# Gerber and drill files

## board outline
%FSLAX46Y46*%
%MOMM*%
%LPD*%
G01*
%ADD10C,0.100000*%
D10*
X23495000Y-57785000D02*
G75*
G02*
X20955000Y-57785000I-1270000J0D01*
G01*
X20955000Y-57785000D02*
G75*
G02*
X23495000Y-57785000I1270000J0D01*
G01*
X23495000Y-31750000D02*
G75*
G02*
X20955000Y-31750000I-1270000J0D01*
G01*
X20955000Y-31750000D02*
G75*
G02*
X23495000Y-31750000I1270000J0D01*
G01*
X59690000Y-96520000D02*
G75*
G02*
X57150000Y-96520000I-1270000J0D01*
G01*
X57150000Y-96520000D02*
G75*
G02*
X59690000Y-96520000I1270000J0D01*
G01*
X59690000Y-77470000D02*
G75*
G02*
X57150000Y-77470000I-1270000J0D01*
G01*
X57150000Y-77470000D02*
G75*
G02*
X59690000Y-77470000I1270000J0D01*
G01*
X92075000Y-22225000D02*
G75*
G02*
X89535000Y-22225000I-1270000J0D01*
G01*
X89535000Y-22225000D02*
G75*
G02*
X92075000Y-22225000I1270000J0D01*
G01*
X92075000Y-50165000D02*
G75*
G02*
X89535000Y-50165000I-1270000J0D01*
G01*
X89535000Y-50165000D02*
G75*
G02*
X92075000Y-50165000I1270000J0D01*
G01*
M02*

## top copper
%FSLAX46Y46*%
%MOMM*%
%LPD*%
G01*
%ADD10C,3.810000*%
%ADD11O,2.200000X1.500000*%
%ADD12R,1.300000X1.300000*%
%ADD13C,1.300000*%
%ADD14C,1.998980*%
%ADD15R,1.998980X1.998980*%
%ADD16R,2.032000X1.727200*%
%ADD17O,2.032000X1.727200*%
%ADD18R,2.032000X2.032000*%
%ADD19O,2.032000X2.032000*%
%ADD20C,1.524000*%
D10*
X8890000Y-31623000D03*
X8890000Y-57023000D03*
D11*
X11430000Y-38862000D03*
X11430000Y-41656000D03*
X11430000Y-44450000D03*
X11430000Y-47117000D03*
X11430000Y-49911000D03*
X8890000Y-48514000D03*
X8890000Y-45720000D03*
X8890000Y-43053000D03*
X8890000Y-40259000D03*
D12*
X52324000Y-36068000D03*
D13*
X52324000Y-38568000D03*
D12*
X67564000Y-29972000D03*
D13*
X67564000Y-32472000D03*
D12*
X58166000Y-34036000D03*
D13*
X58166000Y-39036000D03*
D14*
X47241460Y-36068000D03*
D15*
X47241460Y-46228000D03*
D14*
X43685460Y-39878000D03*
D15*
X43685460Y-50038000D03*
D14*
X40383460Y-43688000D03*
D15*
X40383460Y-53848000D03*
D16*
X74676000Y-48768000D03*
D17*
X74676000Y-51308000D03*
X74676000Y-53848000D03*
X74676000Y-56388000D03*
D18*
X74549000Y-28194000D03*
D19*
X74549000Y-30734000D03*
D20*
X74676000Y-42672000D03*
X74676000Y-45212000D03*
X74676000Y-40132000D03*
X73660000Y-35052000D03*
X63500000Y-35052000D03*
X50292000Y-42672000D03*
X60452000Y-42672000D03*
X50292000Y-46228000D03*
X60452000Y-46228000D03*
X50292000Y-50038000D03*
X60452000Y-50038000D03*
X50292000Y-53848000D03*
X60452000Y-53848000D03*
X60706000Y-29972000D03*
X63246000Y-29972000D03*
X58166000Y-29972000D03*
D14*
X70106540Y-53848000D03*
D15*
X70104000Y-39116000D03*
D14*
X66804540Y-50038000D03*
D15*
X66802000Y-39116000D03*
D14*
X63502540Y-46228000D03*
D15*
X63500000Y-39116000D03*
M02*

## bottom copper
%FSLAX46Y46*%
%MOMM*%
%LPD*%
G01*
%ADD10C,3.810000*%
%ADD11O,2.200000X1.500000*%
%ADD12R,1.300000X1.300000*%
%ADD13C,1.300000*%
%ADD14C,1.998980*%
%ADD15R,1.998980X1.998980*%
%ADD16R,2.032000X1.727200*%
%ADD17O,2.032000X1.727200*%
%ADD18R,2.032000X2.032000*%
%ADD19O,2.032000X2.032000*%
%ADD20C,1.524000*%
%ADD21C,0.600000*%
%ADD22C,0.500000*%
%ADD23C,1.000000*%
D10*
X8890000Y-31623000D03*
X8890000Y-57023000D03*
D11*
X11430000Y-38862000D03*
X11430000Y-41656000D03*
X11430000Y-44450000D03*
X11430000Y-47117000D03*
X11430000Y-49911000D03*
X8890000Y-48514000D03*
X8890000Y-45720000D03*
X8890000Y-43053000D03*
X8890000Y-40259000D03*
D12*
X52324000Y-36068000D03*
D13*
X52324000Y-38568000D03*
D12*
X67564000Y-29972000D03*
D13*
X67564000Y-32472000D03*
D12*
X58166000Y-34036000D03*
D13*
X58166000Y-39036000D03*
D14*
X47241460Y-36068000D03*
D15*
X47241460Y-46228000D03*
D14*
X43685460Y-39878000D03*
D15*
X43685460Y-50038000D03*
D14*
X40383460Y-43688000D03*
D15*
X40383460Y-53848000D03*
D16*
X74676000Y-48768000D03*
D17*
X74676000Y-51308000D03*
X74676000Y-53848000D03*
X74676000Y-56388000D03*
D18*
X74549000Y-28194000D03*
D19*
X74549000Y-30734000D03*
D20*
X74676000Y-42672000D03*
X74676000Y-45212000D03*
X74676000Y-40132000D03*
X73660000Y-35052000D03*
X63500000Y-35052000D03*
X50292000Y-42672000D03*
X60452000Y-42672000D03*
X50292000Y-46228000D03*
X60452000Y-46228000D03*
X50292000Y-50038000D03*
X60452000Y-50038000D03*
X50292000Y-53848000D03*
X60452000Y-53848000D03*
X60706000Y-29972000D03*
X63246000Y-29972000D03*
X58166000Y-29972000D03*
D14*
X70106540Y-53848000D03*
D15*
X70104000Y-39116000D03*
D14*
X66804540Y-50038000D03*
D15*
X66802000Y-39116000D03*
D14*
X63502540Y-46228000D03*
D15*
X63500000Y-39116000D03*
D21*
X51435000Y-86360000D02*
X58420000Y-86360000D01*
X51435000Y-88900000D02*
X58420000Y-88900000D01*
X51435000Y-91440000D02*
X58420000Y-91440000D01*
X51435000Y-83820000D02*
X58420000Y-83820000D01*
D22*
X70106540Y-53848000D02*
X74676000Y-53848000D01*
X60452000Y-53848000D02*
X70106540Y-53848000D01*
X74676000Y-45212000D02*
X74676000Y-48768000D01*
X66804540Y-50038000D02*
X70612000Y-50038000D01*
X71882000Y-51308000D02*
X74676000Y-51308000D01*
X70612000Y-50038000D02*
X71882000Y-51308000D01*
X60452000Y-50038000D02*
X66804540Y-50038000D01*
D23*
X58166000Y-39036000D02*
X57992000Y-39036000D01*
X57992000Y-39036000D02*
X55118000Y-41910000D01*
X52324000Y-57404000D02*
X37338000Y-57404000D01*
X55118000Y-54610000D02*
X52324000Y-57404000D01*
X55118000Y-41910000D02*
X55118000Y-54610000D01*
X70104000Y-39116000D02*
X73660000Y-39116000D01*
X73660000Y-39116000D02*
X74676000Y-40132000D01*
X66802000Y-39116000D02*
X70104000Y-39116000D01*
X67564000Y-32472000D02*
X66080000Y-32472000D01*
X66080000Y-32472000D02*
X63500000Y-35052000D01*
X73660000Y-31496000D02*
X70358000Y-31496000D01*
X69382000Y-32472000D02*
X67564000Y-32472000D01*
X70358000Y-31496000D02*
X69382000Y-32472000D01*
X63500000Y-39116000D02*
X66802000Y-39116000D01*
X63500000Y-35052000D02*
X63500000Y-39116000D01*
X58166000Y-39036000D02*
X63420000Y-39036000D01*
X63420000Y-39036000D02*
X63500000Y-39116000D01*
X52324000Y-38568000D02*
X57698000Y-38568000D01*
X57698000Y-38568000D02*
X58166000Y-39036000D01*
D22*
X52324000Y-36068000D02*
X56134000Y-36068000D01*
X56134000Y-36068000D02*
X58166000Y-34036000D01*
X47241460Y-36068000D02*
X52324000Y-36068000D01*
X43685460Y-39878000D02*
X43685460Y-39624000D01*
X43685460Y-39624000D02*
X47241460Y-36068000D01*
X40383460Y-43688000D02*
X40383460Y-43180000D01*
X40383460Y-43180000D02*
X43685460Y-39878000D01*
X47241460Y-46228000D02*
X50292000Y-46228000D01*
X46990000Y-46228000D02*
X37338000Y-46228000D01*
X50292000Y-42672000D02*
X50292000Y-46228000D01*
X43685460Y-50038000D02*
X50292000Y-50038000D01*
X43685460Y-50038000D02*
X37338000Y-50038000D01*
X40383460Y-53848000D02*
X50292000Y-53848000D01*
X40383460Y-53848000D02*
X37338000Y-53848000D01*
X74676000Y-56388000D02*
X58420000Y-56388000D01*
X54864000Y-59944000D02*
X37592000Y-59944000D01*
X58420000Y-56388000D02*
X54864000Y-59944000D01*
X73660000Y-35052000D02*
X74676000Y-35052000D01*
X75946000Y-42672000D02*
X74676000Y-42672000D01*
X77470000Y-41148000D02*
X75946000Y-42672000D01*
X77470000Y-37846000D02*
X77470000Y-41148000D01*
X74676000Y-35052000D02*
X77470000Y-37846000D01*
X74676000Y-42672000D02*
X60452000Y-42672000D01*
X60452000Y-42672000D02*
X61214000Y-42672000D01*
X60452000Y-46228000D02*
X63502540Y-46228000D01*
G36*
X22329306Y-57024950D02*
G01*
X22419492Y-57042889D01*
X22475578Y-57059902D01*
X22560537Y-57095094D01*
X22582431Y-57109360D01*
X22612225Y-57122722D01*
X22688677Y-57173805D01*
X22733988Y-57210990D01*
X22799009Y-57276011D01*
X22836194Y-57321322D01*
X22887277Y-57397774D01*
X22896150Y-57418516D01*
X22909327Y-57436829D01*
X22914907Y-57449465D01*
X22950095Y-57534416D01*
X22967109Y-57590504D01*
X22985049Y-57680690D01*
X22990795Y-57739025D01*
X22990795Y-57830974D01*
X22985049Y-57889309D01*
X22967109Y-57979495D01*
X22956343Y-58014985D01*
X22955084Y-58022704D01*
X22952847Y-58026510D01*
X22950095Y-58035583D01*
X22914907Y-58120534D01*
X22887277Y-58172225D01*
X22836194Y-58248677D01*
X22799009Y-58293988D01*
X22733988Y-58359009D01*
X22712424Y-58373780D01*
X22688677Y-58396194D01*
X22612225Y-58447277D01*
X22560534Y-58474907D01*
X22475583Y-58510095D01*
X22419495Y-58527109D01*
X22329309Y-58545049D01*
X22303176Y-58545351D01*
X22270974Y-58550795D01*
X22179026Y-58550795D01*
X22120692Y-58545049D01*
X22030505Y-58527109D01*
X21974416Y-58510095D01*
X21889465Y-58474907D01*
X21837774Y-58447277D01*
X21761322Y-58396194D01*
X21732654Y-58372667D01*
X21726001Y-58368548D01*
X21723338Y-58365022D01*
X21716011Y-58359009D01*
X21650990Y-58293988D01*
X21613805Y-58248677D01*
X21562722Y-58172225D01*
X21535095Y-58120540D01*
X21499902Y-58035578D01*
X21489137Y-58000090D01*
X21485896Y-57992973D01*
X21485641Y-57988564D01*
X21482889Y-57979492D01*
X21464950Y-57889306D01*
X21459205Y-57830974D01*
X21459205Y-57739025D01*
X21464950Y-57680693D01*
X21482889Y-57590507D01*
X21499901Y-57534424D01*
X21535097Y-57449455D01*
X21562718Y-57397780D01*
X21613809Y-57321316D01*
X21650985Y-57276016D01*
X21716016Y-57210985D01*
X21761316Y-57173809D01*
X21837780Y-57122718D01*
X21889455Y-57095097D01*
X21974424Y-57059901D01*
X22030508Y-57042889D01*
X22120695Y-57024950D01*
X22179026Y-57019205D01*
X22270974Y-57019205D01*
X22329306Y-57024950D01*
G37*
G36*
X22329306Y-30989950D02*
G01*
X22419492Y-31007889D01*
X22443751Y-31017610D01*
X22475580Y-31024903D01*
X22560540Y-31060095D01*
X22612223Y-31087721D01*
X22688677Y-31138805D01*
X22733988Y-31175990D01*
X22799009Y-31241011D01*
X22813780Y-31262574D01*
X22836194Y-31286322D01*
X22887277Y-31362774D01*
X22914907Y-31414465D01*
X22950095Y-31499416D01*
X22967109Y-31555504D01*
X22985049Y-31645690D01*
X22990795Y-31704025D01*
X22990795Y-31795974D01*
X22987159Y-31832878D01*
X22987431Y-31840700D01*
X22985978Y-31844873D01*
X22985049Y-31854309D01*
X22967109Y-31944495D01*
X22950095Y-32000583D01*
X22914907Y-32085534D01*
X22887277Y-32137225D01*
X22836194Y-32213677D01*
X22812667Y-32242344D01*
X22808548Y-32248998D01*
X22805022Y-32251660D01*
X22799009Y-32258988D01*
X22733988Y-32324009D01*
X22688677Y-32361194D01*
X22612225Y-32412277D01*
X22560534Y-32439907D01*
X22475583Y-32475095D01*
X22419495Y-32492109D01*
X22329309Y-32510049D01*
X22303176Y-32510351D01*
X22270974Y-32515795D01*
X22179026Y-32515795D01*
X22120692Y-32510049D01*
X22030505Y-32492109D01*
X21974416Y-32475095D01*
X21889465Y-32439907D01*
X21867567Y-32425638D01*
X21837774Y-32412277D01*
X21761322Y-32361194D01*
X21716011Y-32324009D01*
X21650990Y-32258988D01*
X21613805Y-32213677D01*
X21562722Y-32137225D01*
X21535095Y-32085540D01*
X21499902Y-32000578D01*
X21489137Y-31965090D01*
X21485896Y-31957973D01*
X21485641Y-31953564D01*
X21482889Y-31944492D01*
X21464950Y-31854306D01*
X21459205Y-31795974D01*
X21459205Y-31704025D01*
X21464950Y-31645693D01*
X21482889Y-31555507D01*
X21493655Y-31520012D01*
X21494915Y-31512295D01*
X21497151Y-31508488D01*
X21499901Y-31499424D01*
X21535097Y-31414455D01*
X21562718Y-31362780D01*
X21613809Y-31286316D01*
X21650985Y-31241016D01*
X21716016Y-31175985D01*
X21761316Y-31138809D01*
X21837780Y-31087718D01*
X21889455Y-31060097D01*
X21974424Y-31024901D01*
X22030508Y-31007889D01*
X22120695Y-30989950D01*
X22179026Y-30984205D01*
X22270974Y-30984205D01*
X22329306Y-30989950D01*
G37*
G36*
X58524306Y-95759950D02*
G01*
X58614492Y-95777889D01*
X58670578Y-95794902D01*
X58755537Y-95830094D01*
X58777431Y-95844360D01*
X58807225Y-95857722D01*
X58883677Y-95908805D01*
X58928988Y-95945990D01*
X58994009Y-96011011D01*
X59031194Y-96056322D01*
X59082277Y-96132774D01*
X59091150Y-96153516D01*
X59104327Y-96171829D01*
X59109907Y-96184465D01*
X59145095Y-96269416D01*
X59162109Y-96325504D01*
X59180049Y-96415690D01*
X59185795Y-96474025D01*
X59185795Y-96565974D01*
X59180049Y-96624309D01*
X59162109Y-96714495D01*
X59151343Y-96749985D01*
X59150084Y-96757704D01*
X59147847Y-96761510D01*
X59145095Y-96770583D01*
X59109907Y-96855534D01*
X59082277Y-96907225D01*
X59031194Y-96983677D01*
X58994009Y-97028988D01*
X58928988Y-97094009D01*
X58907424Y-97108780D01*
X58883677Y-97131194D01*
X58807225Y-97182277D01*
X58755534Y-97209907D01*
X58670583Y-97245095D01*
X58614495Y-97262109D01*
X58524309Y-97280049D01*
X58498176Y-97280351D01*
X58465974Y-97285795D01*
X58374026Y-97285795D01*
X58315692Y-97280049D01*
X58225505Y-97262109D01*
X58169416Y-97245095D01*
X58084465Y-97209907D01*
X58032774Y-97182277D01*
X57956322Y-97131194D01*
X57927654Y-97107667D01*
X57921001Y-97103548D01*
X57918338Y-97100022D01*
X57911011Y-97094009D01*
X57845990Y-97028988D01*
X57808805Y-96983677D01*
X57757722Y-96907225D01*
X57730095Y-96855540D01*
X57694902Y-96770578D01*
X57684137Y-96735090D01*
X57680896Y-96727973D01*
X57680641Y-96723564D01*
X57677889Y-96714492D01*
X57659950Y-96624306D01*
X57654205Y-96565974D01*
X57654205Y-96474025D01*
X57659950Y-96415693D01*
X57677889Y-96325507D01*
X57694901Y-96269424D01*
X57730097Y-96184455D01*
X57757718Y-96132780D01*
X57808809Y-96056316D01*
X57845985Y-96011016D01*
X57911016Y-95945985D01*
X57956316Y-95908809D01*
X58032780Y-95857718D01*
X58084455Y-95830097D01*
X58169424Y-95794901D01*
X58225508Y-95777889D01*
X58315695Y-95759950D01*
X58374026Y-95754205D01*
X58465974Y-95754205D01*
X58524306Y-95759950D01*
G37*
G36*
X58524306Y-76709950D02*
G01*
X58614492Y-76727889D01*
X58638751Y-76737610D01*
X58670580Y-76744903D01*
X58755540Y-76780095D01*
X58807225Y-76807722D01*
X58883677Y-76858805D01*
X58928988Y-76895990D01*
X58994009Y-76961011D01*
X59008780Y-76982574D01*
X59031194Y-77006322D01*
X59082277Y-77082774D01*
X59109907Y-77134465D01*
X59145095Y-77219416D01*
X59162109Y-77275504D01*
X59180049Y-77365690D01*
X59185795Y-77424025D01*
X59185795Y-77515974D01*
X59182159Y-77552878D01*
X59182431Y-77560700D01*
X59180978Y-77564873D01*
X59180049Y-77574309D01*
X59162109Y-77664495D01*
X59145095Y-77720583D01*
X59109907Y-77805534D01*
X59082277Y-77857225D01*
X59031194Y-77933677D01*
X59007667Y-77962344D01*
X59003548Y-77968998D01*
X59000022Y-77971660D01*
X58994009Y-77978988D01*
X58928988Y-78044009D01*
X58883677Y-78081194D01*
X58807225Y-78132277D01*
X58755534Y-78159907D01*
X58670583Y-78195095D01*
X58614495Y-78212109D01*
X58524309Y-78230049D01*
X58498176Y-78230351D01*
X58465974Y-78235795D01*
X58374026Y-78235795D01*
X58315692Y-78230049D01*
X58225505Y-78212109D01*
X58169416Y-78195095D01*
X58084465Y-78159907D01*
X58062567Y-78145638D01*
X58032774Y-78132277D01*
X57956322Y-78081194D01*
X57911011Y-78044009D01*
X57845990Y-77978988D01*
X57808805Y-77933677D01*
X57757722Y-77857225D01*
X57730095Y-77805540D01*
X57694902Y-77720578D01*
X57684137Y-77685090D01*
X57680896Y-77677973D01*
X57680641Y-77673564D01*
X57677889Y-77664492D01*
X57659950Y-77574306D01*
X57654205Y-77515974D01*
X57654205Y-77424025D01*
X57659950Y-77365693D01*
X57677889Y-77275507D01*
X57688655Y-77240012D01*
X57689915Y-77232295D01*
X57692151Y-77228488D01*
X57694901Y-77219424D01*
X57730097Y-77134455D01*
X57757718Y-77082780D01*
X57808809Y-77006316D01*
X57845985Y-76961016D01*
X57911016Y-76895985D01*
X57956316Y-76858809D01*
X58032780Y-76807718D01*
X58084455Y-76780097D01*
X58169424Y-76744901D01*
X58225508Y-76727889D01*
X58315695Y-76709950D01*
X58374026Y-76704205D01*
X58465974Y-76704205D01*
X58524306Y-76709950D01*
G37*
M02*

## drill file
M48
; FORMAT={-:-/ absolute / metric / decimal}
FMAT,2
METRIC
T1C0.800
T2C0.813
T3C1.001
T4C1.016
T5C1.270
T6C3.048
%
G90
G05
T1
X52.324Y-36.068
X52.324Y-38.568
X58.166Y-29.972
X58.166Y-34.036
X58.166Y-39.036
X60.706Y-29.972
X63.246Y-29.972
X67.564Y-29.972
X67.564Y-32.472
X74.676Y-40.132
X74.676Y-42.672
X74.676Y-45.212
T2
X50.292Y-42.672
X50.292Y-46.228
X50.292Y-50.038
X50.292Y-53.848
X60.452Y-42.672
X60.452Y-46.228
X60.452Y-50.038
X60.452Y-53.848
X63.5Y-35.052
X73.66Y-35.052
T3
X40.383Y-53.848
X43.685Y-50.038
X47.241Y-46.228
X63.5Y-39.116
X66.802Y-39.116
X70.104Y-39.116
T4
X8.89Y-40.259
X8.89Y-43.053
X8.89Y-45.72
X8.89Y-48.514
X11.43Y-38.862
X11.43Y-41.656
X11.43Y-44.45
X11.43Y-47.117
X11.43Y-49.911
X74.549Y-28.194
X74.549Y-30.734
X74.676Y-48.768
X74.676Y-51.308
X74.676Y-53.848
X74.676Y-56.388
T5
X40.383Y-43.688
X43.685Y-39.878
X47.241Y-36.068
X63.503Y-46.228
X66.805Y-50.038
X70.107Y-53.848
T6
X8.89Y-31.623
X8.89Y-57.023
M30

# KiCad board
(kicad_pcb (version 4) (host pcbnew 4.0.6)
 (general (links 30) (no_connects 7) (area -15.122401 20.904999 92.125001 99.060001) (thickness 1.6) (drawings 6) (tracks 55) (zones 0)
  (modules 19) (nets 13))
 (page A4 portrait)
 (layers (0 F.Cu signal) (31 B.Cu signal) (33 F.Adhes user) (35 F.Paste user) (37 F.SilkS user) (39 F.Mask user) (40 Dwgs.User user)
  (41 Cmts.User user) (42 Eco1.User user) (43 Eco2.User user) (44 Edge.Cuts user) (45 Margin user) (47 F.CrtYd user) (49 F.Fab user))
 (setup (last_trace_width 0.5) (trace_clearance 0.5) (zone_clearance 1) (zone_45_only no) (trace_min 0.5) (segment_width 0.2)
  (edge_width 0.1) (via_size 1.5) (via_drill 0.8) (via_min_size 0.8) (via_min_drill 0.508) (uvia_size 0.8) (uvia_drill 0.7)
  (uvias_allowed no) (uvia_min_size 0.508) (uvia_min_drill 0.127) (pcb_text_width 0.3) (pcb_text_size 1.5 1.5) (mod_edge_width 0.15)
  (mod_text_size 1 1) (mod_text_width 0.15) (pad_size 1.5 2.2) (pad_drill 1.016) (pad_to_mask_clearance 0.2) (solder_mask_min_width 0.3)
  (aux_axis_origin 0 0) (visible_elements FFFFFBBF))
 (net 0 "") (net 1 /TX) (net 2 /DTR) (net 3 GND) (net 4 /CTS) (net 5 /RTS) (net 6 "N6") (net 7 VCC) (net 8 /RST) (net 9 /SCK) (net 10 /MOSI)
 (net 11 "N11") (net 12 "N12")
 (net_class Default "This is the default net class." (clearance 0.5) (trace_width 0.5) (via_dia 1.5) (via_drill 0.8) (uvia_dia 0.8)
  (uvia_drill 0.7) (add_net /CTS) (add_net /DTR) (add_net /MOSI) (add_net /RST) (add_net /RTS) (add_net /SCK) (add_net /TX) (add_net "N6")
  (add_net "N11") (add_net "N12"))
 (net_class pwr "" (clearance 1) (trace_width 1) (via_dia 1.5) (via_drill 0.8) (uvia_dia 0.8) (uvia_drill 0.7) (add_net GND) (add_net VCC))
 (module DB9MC (layer F.Cu) (at 10.16 44.45 90)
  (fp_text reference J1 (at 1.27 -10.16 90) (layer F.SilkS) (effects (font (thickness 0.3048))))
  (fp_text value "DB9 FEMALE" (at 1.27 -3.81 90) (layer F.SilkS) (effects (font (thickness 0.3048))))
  (pad "" thru_hole circle (at 12.827 -1.27 90) (size 3.81 3.81) (drill 3.048) (layers *.Cu *.Mask F.SilkS))
  (pad "" thru_hole circle (at -12.573 -1.27 90) (size 3.81 3.81) (drill 3.048) (layers *.Cu *.Mask F.SilkS))
  (pad 1 thru_hole oval (at 5.588 1.27 90) (size 1.5 2.2) (drill 1.016) (layers *.Cu *.Mask F.SilkS))
  (pad 2 thru_hole oval (at 2.794 1.27 90) (size 1.5 2.2) (drill 1.016) (layers *.Cu *.Mask F.SilkS))
  (pad 3 thru_hole oval (at 0 1.27 90) (size 1.5 2.2) (drill 1.016) (layers *.Cu *.Mask F.SilkS) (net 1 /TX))
  (pad 4 thru_hole oval (at -2.667 1.27 90) (size 1.5 2.2) (drill 1.016) (layers *.Cu *.Mask F.SilkS) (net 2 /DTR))
  (pad 5 thru_hole oval (at -5.461 1.27 90) (size 1.5 2.2) (drill 1.016) (layers *.Cu *.Mask F.SilkS) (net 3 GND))
  (pad 9 thru_hole oval (at -4.064 -1.27 90) (size 1.5 2.2) (drill 1.016) (layers *.Cu *.Mask F.SilkS))
  (pad 8 thru_hole oval (at -1.27 -1.27 90) (size 1.5 2.2) (drill 1.016) (layers *.Cu *.Mask F.SilkS) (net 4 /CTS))
  (pad 7 thru_hole oval (at 1.397 -1.27 90) (size 1.5 2.2) (drill 1.016) (layers *.Cu *.Mask F.SilkS) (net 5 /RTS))
  (pad 6 thru_hole oval (at 4.191 -1.27 90) (size 1.5 2.2) (drill 1.016) (layers *.Cu *.Mask F.SilkS)))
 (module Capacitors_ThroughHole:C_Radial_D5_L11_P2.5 (layer F.Cu) (at 52.324 36.068 270)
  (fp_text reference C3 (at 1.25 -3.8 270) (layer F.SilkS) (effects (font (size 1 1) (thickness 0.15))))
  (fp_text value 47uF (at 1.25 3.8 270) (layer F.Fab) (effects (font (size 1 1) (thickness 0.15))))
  (pad 1 thru_hole rect (at 0 0 270) (size 1.3 1.3) (drill 0.8) (layers *.Cu *.Mask F.SilkS) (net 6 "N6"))
  (pad 2 thru_hole circle (at 2.5 0 270) (size 1.3 1.3) (drill 0.8) (layers *.Cu *.Mask F.SilkS) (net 3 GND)))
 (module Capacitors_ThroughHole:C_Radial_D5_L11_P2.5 (layer F.Cu) (at 67.564 29.972 270)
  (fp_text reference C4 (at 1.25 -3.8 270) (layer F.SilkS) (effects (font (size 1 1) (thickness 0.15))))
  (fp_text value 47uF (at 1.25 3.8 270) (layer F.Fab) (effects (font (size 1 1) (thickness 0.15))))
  (pad 1 thru_hole rect (at 0 0 270) (size 1.3 1.3) (drill 0.8) (layers *.Cu *.Mask F.SilkS) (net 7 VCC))
  (pad 2 thru_hole circle (at 2.5 0 270) (size 1.3 1.3) (drill 0.8) (layers *.Cu *.Mask F.SilkS) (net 3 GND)))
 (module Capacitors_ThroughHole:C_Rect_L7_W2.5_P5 (layer F.Cu) (at 58.166 34.036 270)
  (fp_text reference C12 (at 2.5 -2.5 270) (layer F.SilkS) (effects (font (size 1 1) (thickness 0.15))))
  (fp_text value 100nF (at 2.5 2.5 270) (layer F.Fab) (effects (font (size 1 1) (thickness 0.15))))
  (pad 1 thru_hole rect (at 0 0 270) (size 1.3 1.3) (drill 0.8) (layers *.Cu *.Mask F.SilkS) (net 6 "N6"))
  (pad 2 thru_hole circle (at 5 0 270) (size 1.3 1.3) (drill 0.8) (layers *.Cu *.Mask F.SilkS) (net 3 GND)))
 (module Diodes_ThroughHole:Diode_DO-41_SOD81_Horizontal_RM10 (layer F.Cu) (at 47.244 46.228 90)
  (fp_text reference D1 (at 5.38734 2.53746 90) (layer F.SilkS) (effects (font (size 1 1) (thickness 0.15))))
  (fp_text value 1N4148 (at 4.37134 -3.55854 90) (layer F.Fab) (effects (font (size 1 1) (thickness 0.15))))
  (pad 2 thru_hole circle (at 10.16 -0.00254 270) (size 1.99898 1.99898) (drill 1.27) (layers *.Cu *.Mask F.SilkS) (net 6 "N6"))
  (pad 1 thru_hole rect (at 0 -0.00254 270) (size 1.99898 1.99898) (drill 1.00076) (layers *.Cu *.Mask F.SilkS) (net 1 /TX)))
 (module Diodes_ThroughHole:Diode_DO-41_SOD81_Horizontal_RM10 (layer F.Cu) (at 43.688 50.038 90)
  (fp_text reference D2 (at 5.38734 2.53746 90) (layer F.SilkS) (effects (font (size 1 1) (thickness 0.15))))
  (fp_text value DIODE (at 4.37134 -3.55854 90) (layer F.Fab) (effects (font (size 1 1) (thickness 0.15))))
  (pad 2 thru_hole circle (at 10.16 -0.00254 270) (size 1.99898 1.99898) (drill 1.27) (layers *.Cu *.Mask F.SilkS) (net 6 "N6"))
  (pad 1 thru_hole rect (at 0 -0.00254 270) (size 1.99898 1.99898) (drill 1.00076) (layers *.Cu *.Mask F.SilkS) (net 5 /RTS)))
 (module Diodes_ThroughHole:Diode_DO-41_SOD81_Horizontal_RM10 (layer F.Cu) (at 40.386 53.848 90)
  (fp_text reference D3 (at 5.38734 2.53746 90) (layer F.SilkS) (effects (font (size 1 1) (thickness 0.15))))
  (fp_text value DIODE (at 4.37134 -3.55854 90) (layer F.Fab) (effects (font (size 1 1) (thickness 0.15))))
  (pad 2 thru_hole circle (at 10.16 -0.00254 270) (size 1.99898 1.99898) (drill 1.27) (layers *.Cu *.Mask F.SilkS) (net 6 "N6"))
  (pad 1 thru_hole rect (at 0 -0.00254 270) (size 1.99898 1.99898) (drill 1.00076) (layers *.Cu *.Mask F.SilkS) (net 2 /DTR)))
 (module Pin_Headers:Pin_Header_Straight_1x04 (layer F.Cu) (at 74.676 48.768)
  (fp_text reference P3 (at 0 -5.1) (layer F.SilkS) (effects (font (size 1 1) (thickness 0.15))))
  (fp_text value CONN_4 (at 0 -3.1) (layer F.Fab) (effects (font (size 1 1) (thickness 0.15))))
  (pad 1 thru_hole rect (at 0 0) (size 2.032 1.7272) (drill 1.016) (layers *.Cu *.Mask F.SilkS) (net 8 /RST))
  (pad 2 thru_hole oval (at 0 2.54) (size 2.032 1.7272) (drill 1.016) (layers *.Cu *.Mask F.SilkS) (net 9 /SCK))
  (pad 3 thru_hole oval (at 0 5.08) (size 2.032 1.7272) (drill 1.016) (layers *.Cu *.Mask F.SilkS) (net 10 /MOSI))
  (pad 4 thru_hole oval (at 0 7.62) (size 2.032 1.7272) (drill 1.016) (layers *.Cu *.Mask F.SilkS) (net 4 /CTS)))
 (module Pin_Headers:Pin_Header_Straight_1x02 (layer F.Cu) (at 74.549 28.194)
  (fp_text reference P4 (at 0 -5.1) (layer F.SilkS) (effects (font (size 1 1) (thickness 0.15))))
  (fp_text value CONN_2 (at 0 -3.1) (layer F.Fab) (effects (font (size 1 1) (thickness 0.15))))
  (pad 1 thru_hole rect (at 0 0) (size 2.032 2.032) (drill 1.016) (layers *.Cu *.Mask F.SilkS) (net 7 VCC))
  (pad 2 thru_hole oval (at 0 2.54) (size 2.032 2.032) (drill 1.016) (layers *.Cu *.Mask F.SilkS) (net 3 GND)))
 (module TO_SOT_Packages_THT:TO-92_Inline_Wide (layer F.Cu) (at 74.676 40.132 270)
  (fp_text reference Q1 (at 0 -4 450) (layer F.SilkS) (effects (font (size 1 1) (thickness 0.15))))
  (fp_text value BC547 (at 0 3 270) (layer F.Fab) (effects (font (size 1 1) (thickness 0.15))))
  (pad 2 thru_hole circle (at 2.54 0) (size 1.524 1.524) (drill 0.8) (layers *.Cu *.Mask F.SilkS) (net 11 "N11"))
  (pad 3 thru_hole circle (at 5.08 0) (size 1.524 1.524) (drill 0.8) (layers *.Cu *.Mask F.SilkS) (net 8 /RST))
  (pad 1 thru_hole circle (at 0 0) (size 1.524 1.524) (drill 0.8) (layers *.Cu *.Mask F.SilkS) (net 3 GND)))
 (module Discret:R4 (layer F.Cu) (at 68.58 35.052 180)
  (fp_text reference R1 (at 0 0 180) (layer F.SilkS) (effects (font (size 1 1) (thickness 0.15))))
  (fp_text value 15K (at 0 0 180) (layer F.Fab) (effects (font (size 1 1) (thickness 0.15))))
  (pad 1 thru_hole circle (at -5.08 0 180) (size 1.524 1.524) (drill 0.8128) (layers *.Cu *.Mask F.SilkS) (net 11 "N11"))
  (pad 2 thru_hole circle (at 5.08 0 180) (size 1.524 1.524) (drill 0.8128) (layers *.Cu *.Mask F.SilkS) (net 3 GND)))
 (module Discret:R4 (layer F.Cu) (at 55.372 42.672)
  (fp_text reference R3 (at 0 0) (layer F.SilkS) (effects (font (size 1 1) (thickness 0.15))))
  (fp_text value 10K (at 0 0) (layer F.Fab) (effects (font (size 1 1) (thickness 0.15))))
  (pad 1 thru_hole circle (at -5.08 0) (size 1.524 1.524) (drill 0.8128) (layers *.Cu *.Mask F.SilkS) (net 1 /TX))
  (pad 2 thru_hole circle (at 5.08 0) (size 1.524 1.524) (drill 0.8128) (layers *.Cu *.Mask F.SilkS) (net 11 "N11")))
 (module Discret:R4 (layer F.Cu) (at 55.372 46.228)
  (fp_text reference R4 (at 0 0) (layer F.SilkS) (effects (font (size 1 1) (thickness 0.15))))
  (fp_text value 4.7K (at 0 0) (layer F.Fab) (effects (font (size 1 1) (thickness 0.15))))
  (pad 1 thru_hole circle (at -5.08 0) (size 1.524 1.524) (drill 0.8128) (layers *.Cu *.Mask F.SilkS) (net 1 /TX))
  (pad 2 thru_hole circle (at 5.08 0) (size 1.524 1.524) (drill 0.8128) (layers *.Cu *.Mask F.SilkS) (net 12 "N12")))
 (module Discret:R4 (layer F.Cu) (at 55.372 50.038)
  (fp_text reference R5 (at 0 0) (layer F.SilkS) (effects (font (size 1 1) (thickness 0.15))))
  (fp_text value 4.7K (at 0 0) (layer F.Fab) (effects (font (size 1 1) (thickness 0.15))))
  (pad 1 thru_hole circle (at -5.08 0) (size 1.524 1.524) (drill 0.8128) (layers *.Cu *.Mask F.SilkS) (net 5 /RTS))
  (pad 2 thru_hole circle (at 5.08 0) (size 1.524 1.524) (drill 0.8128) (layers *.Cu *.Mask F.SilkS) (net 9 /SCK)))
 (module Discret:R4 (layer F.Cu) (at 55.372 53.848)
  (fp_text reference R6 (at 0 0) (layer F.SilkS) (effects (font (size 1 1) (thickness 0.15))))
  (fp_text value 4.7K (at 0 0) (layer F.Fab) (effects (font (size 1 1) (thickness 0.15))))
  (pad 1 thru_hole circle (at -5.08 0) (size 1.524 1.524) (drill 0.8128) (layers *.Cu *.Mask F.SilkS) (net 2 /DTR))
  (pad 2 thru_hole circle (at 5.08 0) (size 1.524 1.524) (drill 0.8128) (layers *.Cu *.Mask F.SilkS) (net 10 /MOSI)))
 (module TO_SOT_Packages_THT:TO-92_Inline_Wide (layer F.Cu) (at 58.166 29.972)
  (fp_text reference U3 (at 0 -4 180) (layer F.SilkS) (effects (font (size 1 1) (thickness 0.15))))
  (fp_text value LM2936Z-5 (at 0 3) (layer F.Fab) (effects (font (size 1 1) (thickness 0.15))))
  (pad 2 thru_hole circle (at 2.54 0 90) (size 1.524 1.524) (drill 0.8) (layers *.Cu *.Mask F.SilkS))
  (pad 3 thru_hole circle (at 5.08 0 90) (size 1.524 1.524) (drill 0.8) (layers *.Cu *.Mask F.SilkS))
  (pad 1 thru_hole circle (at 0 0 90) (size 1.524 1.524) (drill 0.8) (layers *.Cu *.Mask F.SilkS)))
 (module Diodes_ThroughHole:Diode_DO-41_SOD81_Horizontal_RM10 (layer F.Cu) (at 70.104 43.688 270)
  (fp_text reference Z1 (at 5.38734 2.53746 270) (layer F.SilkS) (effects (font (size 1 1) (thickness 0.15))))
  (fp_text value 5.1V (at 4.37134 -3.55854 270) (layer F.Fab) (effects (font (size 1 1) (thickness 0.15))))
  (pad 2 thru_hole circle (at 10.16 -0.00254 90) (size 1.99898 1.99898) (drill 1.27) (layers *.Cu *.Mask F.SilkS) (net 10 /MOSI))
  (pad 1 thru_hole rect (at -4.572 0 90) (size 1.99898 1.99898) (drill 1.00076) (layers *.Cu *.Mask F.SilkS) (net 3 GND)))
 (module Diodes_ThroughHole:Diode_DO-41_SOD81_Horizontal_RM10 (layer F.Cu) (at 66.802 39.878 270)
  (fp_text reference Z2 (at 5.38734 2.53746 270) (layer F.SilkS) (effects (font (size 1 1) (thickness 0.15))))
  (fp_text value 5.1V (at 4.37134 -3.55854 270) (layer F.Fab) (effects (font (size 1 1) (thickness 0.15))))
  (pad 2 thru_hole circle (at 10.16 -0.00254 90) (size 1.99898 1.99898) (drill 1.27) (layers *.Cu *.Mask F.SilkS) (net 9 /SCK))
  (pad 1 thru_hole rect (at -0.762 0 90) (size 1.99898 1.99898) (drill 1.00076) (layers *.Cu *.Mask F.SilkS) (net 3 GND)))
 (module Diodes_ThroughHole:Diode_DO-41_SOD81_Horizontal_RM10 (layer F.Cu) (at 63.5 36.068 270)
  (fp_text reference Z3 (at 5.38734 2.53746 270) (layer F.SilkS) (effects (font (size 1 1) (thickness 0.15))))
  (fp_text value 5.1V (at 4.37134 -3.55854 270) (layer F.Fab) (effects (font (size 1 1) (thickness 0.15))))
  (pad 2 thru_hole circle (at 10.16 -0.00254 90) (size 1.99898 1.99898) (drill 1.27) (layers *.Cu *.Mask F.SilkS) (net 12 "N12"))
  (pad 1 thru_hole rect (at 3.048 0 90) (size 1.99898 1.99898) (drill 1.00076) (layers *.Cu *.Mask F.SilkS) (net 3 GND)))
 (gr_circle (center 22.225 57.785) (end 23.495 57.785) (layer Edge.Cuts) (width 0.1))
 (gr_circle (center 22.225 31.75) (end 23.495 31.75) (layer Edge.Cuts) (width 0.1))
 (gr_circle (center 58.42 96.52) (end 59.69 96.52) (layer Edge.Cuts) (width 0.1))
 (gr_circle (center 58.42 77.47) (end 59.69 77.47) (layer Edge.Cuts) (width 0.1))
 (gr_circle (center 90.805 22.225) (end 89.535 22.225) (layer Edge.Cuts) (width 0.1))
 (gr_circle (center 90.805 50.165) (end 89.535 50.165) (layer Edge.Cuts) (width 0.1))
 (segment (start 51.435 86.36) (end 58.42 86.36) (width 0.6) (layer B.Cu) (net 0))
 (segment (start 51.435 88.9) (end 58.42 88.9) (width 0.6) (layer B.Cu) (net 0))
 (segment (start 51.435 91.44) (end 58.42 91.44) (width 0.6) (layer B.Cu) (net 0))
 (segment (start 51.435 83.82) (end 58.42 83.82) (width 0.6) (layer B.Cu) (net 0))
 (segment (start 70.10654 53.848) (end 74.676 53.848) (width 0.5) (layer B.Cu) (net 10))
 (segment (start 60.452 53.848) (end 70.10654 53.848) (width 0.5) (layer B.Cu) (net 10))
 (segment (start 74.676 45.212) (end 74.676 48.768) (width 0.5) (layer B.Cu) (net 8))
 (segment (start 66.80454 50.038) (end 70.612 50.038) (width 0.5) (layer B.Cu) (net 9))
 (segment (start 71.882 51.308) (end 74.676 51.308) (width 0.5) (layer B.Cu) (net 9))
 (segment (start 70.612 50.038) (end 71.882 51.308) (width 0.5) (layer B.Cu) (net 9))
 (segment (start 60.452 50.038) (end 66.80454 50.038) (width 0.5) (layer B.Cu) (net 9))
 (segment (start 58.166 39.036) (end 57.992 39.036) (width 1) (layer B.Cu) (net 3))
 (segment (start 57.992 39.036) (end 55.118 41.91) (width 1) (layer B.Cu) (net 3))
 (segment (start 52.324 57.404) (end 37.338 57.404) (width 1) (layer B.Cu) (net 3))
 (segment (start 55.118 54.61) (end 52.324 57.404) (width 1) (layer B.Cu) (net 3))
 (segment (start 55.118 41.91) (end 55.118 54.61) (width 1) (layer B.Cu) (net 3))
 (segment (start 70.104 39.116) (end 73.66 39.116) (width 1) (layer B.Cu) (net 3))
 (segment (start 73.66 39.116) (end 74.676 40.132) (width 1) (layer B.Cu) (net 3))
 (segment (start 66.802 39.116) (end 70.104 39.116) (width 1) (layer B.Cu) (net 3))
 (segment (start 67.564 32.472) (end 66.08 32.472) (width 1) (layer B.Cu) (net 3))
 (segment (start 66.08 32.472) (end 63.5 35.052) (width 1) (layer B.Cu) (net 3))
 (segment (start 73.66 31.496) (end 70.358 31.496) (width 1) (layer B.Cu) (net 3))
 (segment (start 69.382 32.472) (end 67.564 32.472) (width 1) (layer B.Cu) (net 3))
 (segment (start 70.358 31.496) (end 69.382 32.472) (width 1) (layer B.Cu) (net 3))
 (segment (start 63.5 39.116) (end 66.802 39.116) (width 1) (layer B.Cu) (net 3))
 (segment (start 63.5 35.052) (end 63.5 39.116) (width 1) (layer B.Cu) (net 3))
 (segment (start 58.166 39.036) (end 63.42 39.036) (width 1) (layer B.Cu) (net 3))
 (segment (start 63.42 39.036) (end 63.5 39.116) (width 1) (layer B.Cu) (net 3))
 (segment (start 52.324 38.568) (end 57.698 38.568) (width 1) (layer B.Cu) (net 3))
 (segment (start 57.698 38.568) (end 58.166 39.036) (width 1) (layer B.Cu) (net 3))
 (segment (start 52.324 36.068) (end 56.134 36.068) (width 0.5) (layer B.Cu) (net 6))
 (segment (start 56.134 36.068) (end 58.166 34.036) (width 0.5) (layer B.Cu) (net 6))
 (segment (start 47.24146 36.068) (end 52.324 36.068) (width 0.5) (layer B.Cu) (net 6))
 (segment (start 43.68546 39.878) (end 43.68546 39.624) (width 0.5) (layer B.Cu) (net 6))
 (segment (start 43.68546 39.624) (end 47.24146 36.068) (width 0.5) (layer B.Cu) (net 6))
 (segment (start 40.38346 43.688) (end 40.38346 43.18) (width 0.5) (layer B.Cu) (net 6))
 (segment (start 40.38346 43.18) (end 43.68546 39.878) (width 0.5) (layer B.Cu) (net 6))
 (segment (start 47.24146 46.228) (end 50.292 46.228) (width 0.5) (layer B.Cu) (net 1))
 (segment (start 46.99 46.228) (end 37.338 46.228) (width 0.5) (layer B.Cu) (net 1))
 (segment (start 50.292 42.672) (end 50.292 46.228) (width 0.5) (layer B.Cu) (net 1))
 (segment (start 43.68546 50.038) (end 50.292 50.038) (width 0.5) (layer B.Cu) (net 5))
 (segment (start 43.68546 50.038) (end 37.338 50.038) (width 0.5) (layer B.Cu) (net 5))
 (segment (start 40.38346 53.848) (end 50.292 53.848) (width 0.5) (layer B.Cu) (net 2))
 (segment (start 40.38346 53.848) (end 37.338 53.848) (width 0.5) (layer B.Cu) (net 2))
 (segment (start 74.676 56.388) (end 58.42 56.388) (width 0.5) (layer B.Cu) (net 4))
 (segment (start 54.864 59.944) (end 37.592 59.944) (width 0.5) (layer B.Cu) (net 4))
 (segment (start 58.42 56.388) (end 54.864 59.944) (width 0.5) (layer B.Cu) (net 4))
 (segment (start 73.66 35.052) (end 74.676 35.052) (width 0.5) (layer B.Cu) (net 11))
 (segment (start 75.946 42.672) (end 74.676 42.672) (width 0.5) (layer B.Cu) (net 11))
 (segment (start 77.47 41.148) (end 75.946 42.672) (width 0.5) (layer B.Cu) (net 11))
 (segment (start 77.47 37.846) (end 77.47 41.148) (width 0.5) (layer B.Cu) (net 11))
 (segment (start 74.676 35.052) (end 77.47 37.846) (width 0.5) (layer B.Cu) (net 11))
 (segment (start 74.676 42.672) (end 60.452 42.672) (width 0.5) (layer B.Cu) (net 11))
 (segment (start 60.452 42.672) (end 61.214 42.672) (width 0.5) (layer B.Cu) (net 11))
 (segment (start 60.452 46.228) (end 63.50254 46.228) (width 0.5) (layer B.Cu) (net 12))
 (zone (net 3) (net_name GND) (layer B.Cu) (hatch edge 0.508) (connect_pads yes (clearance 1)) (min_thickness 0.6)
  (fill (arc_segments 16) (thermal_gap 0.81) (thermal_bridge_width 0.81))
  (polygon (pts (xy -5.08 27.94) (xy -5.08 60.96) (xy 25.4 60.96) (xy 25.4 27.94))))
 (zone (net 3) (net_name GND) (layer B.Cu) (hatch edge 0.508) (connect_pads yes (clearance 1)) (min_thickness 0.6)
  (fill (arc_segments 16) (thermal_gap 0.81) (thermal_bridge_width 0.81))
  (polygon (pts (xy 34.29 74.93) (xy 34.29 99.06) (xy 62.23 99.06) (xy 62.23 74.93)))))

